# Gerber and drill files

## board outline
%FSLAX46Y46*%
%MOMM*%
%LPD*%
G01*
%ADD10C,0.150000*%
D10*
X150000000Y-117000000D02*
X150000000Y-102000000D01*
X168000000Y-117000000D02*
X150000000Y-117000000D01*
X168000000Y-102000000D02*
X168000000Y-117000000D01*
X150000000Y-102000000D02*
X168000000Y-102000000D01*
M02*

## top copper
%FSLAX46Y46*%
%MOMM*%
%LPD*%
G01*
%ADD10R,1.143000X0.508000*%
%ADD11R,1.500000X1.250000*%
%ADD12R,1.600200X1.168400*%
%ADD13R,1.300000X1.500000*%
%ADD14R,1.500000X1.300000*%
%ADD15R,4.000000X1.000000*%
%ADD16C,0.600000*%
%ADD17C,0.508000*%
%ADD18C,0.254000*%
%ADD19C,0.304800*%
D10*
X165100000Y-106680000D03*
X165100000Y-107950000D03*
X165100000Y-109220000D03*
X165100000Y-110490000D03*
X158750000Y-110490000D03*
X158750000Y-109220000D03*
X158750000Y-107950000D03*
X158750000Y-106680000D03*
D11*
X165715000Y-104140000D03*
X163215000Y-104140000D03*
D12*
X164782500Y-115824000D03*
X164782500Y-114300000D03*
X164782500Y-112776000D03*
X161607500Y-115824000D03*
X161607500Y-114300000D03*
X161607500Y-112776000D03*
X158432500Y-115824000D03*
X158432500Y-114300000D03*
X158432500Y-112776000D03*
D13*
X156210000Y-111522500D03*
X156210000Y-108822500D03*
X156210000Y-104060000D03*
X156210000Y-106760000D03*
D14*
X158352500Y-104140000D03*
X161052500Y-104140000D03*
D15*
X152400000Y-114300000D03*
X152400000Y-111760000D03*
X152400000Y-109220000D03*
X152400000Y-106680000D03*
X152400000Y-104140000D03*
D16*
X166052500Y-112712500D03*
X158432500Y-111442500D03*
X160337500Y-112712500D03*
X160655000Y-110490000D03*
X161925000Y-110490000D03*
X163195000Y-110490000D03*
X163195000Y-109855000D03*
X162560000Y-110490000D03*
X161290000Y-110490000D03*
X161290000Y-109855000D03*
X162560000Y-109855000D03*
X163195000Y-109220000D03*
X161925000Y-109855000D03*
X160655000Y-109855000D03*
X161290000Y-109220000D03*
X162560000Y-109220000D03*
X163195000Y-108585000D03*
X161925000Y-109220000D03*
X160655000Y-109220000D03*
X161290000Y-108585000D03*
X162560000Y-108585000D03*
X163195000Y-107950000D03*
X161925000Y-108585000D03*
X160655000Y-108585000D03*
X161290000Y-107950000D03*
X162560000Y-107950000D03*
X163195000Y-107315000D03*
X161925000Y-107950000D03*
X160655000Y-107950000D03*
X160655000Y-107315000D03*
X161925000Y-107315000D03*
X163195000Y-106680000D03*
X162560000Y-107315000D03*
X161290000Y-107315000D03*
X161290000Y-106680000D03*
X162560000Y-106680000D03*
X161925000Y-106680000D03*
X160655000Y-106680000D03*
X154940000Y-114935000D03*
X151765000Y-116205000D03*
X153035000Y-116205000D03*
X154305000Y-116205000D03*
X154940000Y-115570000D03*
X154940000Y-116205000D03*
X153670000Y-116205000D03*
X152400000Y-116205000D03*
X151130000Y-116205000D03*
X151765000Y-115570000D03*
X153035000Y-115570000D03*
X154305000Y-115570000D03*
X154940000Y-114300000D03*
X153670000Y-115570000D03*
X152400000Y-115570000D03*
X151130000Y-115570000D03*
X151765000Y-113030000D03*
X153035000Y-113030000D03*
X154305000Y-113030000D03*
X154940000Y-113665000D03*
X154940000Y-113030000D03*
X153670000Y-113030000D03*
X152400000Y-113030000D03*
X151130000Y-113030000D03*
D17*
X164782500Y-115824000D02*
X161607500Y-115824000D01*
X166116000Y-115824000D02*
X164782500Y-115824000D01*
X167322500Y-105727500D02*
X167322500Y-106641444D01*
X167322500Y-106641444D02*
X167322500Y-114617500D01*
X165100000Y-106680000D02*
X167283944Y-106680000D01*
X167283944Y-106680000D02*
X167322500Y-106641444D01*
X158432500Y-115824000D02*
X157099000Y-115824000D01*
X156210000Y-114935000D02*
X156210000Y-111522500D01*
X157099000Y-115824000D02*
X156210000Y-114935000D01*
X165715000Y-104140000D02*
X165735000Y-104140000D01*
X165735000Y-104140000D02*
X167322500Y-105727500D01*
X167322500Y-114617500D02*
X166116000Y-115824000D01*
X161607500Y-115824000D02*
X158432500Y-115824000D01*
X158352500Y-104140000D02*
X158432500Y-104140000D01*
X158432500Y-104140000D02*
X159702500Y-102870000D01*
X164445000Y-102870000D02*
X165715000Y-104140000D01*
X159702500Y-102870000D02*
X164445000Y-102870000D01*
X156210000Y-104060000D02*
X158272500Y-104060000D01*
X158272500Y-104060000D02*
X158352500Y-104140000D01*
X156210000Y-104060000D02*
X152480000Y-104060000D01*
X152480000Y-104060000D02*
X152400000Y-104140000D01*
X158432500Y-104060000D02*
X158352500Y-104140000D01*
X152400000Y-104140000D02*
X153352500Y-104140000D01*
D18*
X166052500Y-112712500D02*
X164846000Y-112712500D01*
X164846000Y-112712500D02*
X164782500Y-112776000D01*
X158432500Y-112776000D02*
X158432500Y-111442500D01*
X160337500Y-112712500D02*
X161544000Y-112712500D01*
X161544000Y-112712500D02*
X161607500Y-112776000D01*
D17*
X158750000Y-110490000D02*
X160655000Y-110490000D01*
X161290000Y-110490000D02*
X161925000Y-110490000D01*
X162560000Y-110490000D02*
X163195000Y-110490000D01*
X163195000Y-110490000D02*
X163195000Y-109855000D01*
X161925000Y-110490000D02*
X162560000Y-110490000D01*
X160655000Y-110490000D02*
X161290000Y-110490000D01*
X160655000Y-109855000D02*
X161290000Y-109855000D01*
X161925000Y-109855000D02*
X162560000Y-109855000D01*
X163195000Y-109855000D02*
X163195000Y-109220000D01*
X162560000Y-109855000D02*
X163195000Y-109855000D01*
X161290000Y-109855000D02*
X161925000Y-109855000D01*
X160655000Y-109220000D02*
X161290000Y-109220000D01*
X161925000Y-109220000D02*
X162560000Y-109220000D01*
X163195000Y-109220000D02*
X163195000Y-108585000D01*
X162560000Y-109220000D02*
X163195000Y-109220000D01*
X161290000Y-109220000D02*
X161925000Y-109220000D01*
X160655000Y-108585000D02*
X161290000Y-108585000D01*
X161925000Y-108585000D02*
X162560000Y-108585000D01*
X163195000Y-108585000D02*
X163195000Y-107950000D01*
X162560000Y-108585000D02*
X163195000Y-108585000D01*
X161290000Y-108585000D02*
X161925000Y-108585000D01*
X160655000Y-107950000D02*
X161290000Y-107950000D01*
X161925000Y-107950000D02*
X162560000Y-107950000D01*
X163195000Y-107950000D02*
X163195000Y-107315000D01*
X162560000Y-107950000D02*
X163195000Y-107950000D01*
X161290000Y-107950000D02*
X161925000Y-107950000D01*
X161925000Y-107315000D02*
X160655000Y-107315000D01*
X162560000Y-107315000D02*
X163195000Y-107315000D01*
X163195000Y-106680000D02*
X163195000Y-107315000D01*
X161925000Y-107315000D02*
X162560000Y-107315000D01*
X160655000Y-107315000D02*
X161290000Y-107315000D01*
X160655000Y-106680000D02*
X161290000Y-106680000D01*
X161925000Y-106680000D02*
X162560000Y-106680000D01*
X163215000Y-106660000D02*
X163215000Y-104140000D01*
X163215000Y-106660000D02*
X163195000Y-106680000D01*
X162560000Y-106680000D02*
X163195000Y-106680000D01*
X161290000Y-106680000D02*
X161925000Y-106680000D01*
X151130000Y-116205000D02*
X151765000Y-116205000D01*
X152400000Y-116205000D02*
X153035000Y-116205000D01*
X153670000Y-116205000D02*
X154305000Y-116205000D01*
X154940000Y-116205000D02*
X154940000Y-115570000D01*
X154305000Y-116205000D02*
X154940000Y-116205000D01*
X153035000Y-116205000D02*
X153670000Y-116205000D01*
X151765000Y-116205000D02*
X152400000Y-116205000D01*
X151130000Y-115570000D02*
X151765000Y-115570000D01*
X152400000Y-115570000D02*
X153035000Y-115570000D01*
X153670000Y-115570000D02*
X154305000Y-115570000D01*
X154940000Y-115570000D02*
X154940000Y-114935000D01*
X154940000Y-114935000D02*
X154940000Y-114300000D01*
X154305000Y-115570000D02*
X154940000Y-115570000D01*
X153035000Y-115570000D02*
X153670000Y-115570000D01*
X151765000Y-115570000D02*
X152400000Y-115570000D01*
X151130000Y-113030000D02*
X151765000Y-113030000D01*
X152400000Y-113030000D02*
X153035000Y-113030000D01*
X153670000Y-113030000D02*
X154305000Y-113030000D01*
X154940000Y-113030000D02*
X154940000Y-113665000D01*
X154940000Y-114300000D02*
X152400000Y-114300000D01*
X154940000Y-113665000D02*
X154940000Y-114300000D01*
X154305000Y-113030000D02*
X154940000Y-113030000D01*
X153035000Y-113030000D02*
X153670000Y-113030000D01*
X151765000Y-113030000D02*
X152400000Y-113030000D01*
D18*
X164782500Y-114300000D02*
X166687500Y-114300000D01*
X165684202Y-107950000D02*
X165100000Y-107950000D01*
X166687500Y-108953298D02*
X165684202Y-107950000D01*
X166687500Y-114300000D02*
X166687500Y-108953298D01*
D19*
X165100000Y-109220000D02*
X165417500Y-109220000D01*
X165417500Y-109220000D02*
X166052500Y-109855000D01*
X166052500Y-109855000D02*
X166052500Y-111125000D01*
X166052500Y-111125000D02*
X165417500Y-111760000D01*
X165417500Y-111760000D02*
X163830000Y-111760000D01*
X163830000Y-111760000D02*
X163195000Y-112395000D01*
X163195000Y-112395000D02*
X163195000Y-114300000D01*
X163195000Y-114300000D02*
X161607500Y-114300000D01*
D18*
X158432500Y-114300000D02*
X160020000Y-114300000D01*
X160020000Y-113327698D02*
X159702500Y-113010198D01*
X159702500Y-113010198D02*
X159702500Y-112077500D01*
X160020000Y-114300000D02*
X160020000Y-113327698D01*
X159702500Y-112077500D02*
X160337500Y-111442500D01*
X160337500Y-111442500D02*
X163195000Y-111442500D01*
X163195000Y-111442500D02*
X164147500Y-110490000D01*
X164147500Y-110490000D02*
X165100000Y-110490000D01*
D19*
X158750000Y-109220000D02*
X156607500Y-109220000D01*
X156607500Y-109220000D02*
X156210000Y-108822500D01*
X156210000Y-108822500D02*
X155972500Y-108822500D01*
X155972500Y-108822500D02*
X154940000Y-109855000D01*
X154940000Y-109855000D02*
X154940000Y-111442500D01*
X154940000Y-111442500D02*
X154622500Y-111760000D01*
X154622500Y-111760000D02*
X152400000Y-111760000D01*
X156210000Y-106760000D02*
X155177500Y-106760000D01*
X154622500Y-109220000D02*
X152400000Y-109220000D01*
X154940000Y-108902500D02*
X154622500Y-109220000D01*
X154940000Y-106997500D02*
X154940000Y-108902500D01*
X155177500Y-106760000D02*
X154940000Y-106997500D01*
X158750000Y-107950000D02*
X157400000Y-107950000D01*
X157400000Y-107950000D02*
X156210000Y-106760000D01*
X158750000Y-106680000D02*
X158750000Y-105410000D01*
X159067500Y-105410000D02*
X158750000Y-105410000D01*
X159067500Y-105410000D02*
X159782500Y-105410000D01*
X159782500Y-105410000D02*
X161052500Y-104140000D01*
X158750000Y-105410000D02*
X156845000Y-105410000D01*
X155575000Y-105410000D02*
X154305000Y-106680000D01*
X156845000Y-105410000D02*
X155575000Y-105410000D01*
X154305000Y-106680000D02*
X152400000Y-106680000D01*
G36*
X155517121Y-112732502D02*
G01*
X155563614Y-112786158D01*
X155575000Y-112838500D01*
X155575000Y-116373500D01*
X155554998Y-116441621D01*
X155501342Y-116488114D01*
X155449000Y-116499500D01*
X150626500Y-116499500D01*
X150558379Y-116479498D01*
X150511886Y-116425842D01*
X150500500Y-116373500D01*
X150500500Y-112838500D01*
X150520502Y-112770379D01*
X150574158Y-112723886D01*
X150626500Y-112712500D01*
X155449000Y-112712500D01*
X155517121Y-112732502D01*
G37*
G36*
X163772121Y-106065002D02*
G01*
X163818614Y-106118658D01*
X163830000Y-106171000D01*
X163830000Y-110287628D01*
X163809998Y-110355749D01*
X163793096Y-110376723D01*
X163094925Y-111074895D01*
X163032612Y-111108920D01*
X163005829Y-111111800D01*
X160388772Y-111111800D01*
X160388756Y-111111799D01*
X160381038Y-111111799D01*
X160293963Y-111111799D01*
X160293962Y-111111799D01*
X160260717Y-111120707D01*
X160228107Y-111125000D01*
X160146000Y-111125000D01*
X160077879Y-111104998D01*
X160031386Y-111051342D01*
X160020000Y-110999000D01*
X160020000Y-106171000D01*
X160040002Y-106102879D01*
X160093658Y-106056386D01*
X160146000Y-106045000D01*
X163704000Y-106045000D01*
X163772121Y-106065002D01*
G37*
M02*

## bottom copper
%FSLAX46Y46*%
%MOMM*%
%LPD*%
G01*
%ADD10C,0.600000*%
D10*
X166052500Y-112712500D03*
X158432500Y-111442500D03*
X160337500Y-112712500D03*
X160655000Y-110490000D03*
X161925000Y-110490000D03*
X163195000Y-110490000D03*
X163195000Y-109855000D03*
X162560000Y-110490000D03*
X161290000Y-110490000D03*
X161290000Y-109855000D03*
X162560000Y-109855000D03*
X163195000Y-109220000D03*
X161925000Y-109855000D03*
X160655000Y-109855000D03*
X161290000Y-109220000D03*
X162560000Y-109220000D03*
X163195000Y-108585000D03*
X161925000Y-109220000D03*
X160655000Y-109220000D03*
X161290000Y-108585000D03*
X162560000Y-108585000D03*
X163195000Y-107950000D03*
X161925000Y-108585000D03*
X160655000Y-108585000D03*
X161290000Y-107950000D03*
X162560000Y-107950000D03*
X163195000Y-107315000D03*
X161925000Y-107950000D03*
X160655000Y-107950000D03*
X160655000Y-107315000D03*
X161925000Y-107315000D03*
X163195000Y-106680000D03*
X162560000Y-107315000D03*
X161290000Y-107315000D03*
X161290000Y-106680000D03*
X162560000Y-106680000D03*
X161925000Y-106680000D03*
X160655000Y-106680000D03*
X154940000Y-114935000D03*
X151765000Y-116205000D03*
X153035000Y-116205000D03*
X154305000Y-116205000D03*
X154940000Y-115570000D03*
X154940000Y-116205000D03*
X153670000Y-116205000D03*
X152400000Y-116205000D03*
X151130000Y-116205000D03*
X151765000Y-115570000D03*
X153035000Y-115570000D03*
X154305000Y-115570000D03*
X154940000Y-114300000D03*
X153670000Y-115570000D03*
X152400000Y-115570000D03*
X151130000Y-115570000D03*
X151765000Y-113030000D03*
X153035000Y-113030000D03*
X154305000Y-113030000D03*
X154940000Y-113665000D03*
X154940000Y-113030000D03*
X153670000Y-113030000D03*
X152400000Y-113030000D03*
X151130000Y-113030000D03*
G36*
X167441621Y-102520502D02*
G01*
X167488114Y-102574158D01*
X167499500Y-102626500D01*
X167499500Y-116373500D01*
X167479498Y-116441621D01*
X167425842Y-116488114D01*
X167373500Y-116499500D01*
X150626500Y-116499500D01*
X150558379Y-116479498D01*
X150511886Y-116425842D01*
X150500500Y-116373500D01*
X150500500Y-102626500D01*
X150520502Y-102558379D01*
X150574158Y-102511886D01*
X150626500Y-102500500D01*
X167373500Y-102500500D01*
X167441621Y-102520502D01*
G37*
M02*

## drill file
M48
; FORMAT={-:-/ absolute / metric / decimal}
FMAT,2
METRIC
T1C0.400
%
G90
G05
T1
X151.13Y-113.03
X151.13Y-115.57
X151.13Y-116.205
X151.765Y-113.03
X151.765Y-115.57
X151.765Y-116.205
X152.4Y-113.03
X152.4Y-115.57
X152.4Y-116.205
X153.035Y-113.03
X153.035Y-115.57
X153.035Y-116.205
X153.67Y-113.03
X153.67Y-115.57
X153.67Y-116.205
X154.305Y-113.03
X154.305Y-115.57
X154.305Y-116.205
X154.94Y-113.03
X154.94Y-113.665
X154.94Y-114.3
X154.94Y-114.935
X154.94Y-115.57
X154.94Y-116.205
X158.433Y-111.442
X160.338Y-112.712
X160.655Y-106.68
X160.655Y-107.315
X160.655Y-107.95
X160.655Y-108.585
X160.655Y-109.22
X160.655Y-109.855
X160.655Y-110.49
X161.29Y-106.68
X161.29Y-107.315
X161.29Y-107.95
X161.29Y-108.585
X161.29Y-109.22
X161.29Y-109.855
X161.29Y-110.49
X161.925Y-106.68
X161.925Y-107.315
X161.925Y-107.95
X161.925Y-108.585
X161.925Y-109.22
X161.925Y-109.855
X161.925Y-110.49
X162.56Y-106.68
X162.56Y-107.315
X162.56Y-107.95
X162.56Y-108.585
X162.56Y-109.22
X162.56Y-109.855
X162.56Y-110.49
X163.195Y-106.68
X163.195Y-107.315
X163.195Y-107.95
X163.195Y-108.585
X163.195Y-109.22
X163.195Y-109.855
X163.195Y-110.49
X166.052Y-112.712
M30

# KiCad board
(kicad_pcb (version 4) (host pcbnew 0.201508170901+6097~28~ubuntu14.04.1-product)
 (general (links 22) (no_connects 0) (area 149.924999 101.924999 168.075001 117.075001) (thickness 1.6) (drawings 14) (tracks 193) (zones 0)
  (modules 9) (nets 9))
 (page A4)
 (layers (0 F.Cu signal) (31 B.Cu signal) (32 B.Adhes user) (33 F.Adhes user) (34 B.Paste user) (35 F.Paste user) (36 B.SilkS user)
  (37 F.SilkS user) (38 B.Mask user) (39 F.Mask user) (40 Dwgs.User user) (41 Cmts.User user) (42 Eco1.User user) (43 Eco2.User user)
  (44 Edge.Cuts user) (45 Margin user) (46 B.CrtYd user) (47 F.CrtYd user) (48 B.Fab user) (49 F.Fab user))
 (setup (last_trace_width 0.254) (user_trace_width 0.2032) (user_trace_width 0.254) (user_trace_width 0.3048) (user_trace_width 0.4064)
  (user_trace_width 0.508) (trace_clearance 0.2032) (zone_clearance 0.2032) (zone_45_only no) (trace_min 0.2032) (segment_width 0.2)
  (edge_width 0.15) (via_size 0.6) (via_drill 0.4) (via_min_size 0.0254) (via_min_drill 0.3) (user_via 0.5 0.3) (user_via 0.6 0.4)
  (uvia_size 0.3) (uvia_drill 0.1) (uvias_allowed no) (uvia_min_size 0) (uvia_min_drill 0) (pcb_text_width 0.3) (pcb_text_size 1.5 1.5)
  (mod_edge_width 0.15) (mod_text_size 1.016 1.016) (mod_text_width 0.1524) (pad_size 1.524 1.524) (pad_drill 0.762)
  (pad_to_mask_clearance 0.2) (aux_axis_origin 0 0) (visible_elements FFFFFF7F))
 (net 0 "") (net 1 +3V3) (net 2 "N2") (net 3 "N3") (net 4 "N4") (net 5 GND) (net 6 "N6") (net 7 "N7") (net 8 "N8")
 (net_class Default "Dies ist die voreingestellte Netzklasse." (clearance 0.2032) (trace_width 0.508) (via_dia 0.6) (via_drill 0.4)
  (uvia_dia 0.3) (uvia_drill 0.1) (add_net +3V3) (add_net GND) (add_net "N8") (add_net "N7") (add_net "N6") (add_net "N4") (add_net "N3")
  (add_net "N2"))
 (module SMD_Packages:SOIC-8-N (layer F.Cu) (at 161.925 108.585 270)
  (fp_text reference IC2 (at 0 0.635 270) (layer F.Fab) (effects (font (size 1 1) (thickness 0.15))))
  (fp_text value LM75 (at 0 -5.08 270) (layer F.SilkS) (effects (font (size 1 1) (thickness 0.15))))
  (pad 8 smd rect (at -1.905 -3.175 270) (size 0.508 1.143) (layers F.Cu F.Paste F.Mask) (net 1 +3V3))
  (pad 7 smd rect (at -0.635 -3.175 270) (size 0.508 1.143) (layers F.Cu F.Paste F.Mask) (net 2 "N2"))
  (pad 6 smd rect (at 0.635 -3.175 270) (size 0.508 1.143) (layers F.Cu F.Paste F.Mask) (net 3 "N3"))
  (pad 5 smd rect (at 1.905 -3.175 270) (size 0.508 1.143) (layers F.Cu F.Paste F.Mask) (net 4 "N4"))
  (pad 4 smd rect (at 1.905 3.175 270) (size 0.508 1.143) (layers F.Cu F.Paste F.Mask) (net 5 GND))
  (pad 3 smd rect (at 0.635 3.175 270) (size 0.508 1.143) (layers F.Cu F.Paste F.Mask) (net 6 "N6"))
  (pad 2 smd rect (at -0.635 3.175 270) (size 0.508 1.143) (layers F.Cu F.Paste F.Mask) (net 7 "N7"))
  (pad 1 smd rect (at -1.905 3.175 270) (size 0.508 1.143) (layers F.Cu F.Paste F.Mask) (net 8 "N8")))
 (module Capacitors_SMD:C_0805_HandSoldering (layer F.Cu) (at 164.465 104.14 180)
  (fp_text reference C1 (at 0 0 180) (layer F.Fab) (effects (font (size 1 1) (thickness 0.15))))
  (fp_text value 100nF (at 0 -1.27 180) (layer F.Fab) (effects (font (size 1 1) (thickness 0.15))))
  (pad 1 smd rect (at -1.25 0 180) (size 1.5 1.25) (layers F.Cu F.Paste F.Mask) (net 1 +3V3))
  (pad 2 smd rect (at 1.25 0 180) (size 1.5 1.25) (layers F.Cu F.Paste F.Mask) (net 5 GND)))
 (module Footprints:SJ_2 (layer F.Cu) (at 164.7825 114.3 90)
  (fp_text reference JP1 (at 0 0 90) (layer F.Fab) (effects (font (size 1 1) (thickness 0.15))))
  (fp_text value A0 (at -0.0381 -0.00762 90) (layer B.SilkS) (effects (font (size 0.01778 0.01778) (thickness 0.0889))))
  (pad 1 smd rect (at -1.524 0 90) (size 1.1684 1.6002) (layers F.Cu F.Paste F.Mask) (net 1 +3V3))
  (pad 2 smd rect (at 0 0 90) (size 1.1684 1.6002) (layers F.Cu F.Paste F.Mask) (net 2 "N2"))
  (pad 3 smd rect (at 1.524 0 90) (size 1.1684 1.6002) (layers F.Cu F.Paste F.Mask) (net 5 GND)))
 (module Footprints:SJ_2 (layer F.Cu) (at 161.6075 114.3 90)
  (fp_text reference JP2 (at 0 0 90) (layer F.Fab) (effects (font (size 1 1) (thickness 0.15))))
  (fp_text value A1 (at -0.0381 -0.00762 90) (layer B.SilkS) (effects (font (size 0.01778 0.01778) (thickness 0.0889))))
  (pad 1 smd rect (at -1.524 0 90) (size 1.1684 1.6002) (layers F.Cu F.Paste F.Mask) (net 1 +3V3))
  (pad 2 smd rect (at 0 0 90) (size 1.1684 1.6002) (layers F.Cu F.Paste F.Mask) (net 3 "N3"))
  (pad 3 smd rect (at 1.524 0 90) (size 1.1684 1.6002) (layers F.Cu F.Paste F.Mask) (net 5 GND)))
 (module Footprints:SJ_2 (layer F.Cu) (at 158.4325 114.3 90)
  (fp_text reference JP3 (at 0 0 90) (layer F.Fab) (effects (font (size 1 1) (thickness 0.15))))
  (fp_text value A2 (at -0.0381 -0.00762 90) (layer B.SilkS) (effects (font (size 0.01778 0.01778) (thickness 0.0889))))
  (pad 1 smd rect (at -1.524 0 90) (size 1.1684 1.6002) (layers F.Cu F.Paste F.Mask) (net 1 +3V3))
  (pad 2 smd rect (at 0 0 90) (size 1.1684 1.6002) (layers F.Cu F.Paste F.Mask) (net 4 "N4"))
  (pad 3 smd rect (at 1.524 0 90) (size 1.1684 1.6002) (layers F.Cu F.Paste F.Mask) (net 5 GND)))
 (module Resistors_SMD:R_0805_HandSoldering (layer F.Cu) (at 156.21 110.1725 90)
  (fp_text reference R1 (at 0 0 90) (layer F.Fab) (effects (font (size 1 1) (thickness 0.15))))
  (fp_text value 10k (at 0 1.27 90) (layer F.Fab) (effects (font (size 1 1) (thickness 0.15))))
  (pad 1 smd rect (at -1.35 0 90) (size 1.5 1.3) (layers F.Cu F.Paste F.Mask) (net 1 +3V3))
  (pad 2 smd rect (at 1.35 0 90) (size 1.5 1.3) (layers F.Cu F.Paste F.Mask) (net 6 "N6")))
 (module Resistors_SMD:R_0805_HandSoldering (layer F.Cu) (at 156.21 105.41 270)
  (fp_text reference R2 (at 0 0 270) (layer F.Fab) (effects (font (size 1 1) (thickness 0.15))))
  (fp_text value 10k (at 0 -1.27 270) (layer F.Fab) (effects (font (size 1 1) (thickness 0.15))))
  (pad 1 smd rect (at -1.35 0 270) (size 1.5 1.3) (layers F.Cu F.Paste F.Mask) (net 1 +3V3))
  (pad 2 smd rect (at 1.35 0 270) (size 1.5 1.3) (layers F.Cu F.Paste F.Mask) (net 7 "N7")))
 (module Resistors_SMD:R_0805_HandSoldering (layer F.Cu) (at 159.7025 104.14)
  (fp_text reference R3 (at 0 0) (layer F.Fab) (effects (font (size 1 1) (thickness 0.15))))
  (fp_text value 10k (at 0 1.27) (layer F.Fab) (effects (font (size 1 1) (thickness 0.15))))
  (pad 1 smd rect (at -1.35 0) (size 1.5 1.3) (layers F.Cu F.Paste F.Mask) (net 1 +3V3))
  (pad 2 smd rect (at 1.35 0) (size 1.5 1.3) (layers F.Cu F.Paste F.Mask) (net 8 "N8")))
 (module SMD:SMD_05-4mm (layer F.Cu) (at 152.4 104.14)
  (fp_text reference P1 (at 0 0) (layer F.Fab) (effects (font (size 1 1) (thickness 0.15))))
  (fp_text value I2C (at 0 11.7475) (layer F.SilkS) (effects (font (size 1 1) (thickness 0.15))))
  (pad 5 connect rect (at 0 10.16) (size 4 1) (layers F.Cu F.Mask) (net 5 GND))
  (pad 4 connect rect (at 0 7.62) (size 4 1) (layers F.Cu F.Mask) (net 6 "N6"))
  (pad 3 connect rect (at 0 5.08) (size 4 1) (layers F.Cu F.Mask) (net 7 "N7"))
  (pad 2 connect rect (at 0 2.54) (size 4 1) (layers F.Cu F.Mask) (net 8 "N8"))
  (pad 1 connect rect (at 0 0) (size 4 1) (layers F.Cu F.Mask) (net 1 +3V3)))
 (gr_line (start 150 117) (end 150 102) (angle 90) (layer Edge.Cuts) (width 0.15))
 (gr_line (start 168 117) (end 150 117) (angle 90) (layer Edge.Cuts) (width 0.15))
 (gr_line (start 168 102) (end 168 117) (angle 90) (layer Edge.Cuts) (width 0.15))
 (gr_line (start 150 102) (end 168 102) (angle 90) (layer Edge.Cuts) (width 0.15))
 (segment (start 164.7825 115.824) (end 161.6075 115.824) (width 0.508) (layer F.Cu) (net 1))
 (segment (start 166.116 115.824) (end 164.7825 115.824) (width 0.508) (layer F.Cu) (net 1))
 (segment (start 167.3225 105.7275) (end 167.3225 106.641444) (width 0.508) (layer F.Cu) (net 1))
 (segment (start 167.3225 106.641444) (end 167.3225 114.6175) (width 0.508) (layer F.Cu) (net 1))
 (segment (start 165.1 106.68) (end 167.283944 106.68) (width 0.508) (layer F.Cu) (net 1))
 (segment (start 167.283944 106.68) (end 167.3225 106.641444) (width 0.508) (layer F.Cu) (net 1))
 (segment (start 158.4325 115.824) (end 157.099 115.824) (width 0.508) (layer F.Cu) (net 1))
 (segment (start 156.21 114.935) (end 156.21 111.5225) (width 0.508) (layer F.Cu) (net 1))
 (segment (start 157.099 115.824) (end 156.21 114.935) (width 0.508) (layer F.Cu) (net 1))
 (segment (start 165.715 104.14) (end 165.735 104.14) (width 0.508) (layer F.Cu) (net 1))
 (segment (start 165.735 104.14) (end 167.3225 105.7275) (width 0.508) (layer F.Cu) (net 1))
 (segment (start 167.3225 114.6175) (end 166.116 115.824) (width 0.508) (layer F.Cu) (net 1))
 (segment (start 161.6075 115.824) (end 158.4325 115.824) (width 0.508) (layer F.Cu) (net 1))
 (segment (start 158.3525 104.14) (end 158.4325 104.14) (width 0.508) (layer F.Cu) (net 1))
 (segment (start 158.4325 104.14) (end 159.7025 102.87) (width 0.508) (layer F.Cu) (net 1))
 (segment (start 164.445 102.87) (end 165.715 104.14) (width 0.508) (layer F.Cu) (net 1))
 (segment (start 159.7025 102.87) (end 164.445 102.87) (width 0.508) (layer F.Cu) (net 1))
 (segment (start 156.21 104.06) (end 158.2725 104.06) (width 0.508) (layer F.Cu) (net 1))
 (segment (start 158.2725 104.06) (end 158.3525 104.14) (width 0.508) (layer F.Cu) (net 1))
 (segment (start 156.21 104.06) (end 152.48 104.06) (width 0.508) (layer F.Cu) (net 1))
 (segment (start 152.48 104.06) (end 152.4 104.14) (width 0.508) (layer F.Cu) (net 1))
 (segment (start 158.4325 104.06) (end 158.3525 104.14) (width 0.508) (layer F.Cu) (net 1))
 (segment (start 152.4 104.14) (end 153.3525 104.14) (width 0.508) (layer F.Cu) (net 1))
 (via (at 166.0525 112.7125) (size 0.6) (drill 0.4) (layers F.Cu B.Cu) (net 5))
 (segment (start 166.0525 112.7125) (end 164.846 112.7125) (width 0.254) (layer F.Cu) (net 5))
 (segment (start 164.846 112.7125) (end 164.7825 112.776) (width 0.254) (layer F.Cu) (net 5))
 (segment (start 158.4325 112.776) (end 158.4325 111.4425) (width 0.254) (layer F.Cu) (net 5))
 (via (at 158.4325 111.4425) (size 0.6) (drill 0.4) (layers F.Cu B.Cu) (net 5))
 (via (at 160.3375 112.7125) (size 0.6) (drill 0.4) (layers F.Cu B.Cu) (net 5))
 (segment (start 160.3375 112.7125) (end 161.544 112.7125) (width 0.254) (layer F.Cu) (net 5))
 (segment (start 161.544 112.7125) (end 161.6075 112.776) (width 0.254) (layer F.Cu) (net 5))
 (segment (start 158.75 110.49) (end 160.655 110.49) (width 0.508) (layer F.Cu) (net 5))
 (via (at 160.655 110.49) (size 0.6) (drill 0.4) (layers F.Cu B.Cu) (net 5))
 (segment (start 161.29 110.49) (end 161.925 110.49) (width 0.508) (layer F.Cu) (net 5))
 (via (at 161.925 110.49) (size 0.6) (drill 0.4) (layers F.Cu B.Cu) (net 5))
 (segment (start 162.56 110.49) (end 163.195 110.49) (width 0.508) (layer F.Cu) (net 5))
 (via (at 163.195 110.49) (size 0.6) (drill 0.4) (layers F.Cu B.Cu) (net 5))
 (via (at 163.195 109.855) (size 0.6) (drill 0.4) (layers F.Cu B.Cu) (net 5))
 (segment (start 163.195 110.49) (end 163.195 109.855) (width 0.508) (layer F.Cu) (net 5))
 (via (at 162.56 110.49) (size 0.6) (drill 0.4) (layers F.Cu B.Cu) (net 5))
 (segment (start 161.925 110.49) (end 162.56 110.49) (width 0.508) (layer F.Cu) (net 5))
 (via (at 161.29 110.49) (size 0.6) (drill 0.4) (layers F.Cu B.Cu) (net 5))
 (segment (start 160.655 110.49) (end 161.29 110.49) (width 0.508) (layer F.Cu) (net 5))
 (segment (start 160.655 109.855) (end 161.29 109.855) (width 0.508) (layer F.Cu) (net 5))
 (via (at 161.29 109.855) (size 0.6) (drill 0.4) (layers F.Cu B.Cu) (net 5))
 (segment (start 161.925 109.855) (end 162.56 109.855) (width 0.508) (layer F.Cu) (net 5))
 (via (at 162.56 109.855) (size 0.6) (drill 0.4) (layers F.Cu B.Cu) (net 5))
 (segment (start 163.195 109.855) (end 163.195 109.22) (width 0.508) (layer F.Cu) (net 5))
 (via (at 163.195 109.22) (size 0.6) (drill 0.4) (layers F.Cu B.Cu) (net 5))
 (segment (start 162.56 109.855) (end 163.195 109.855) (width 0.508) (layer F.Cu) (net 5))
 (via (at 161.925 109.855) (size 0.6) (drill 0.4) (layers F.Cu B.Cu) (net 5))
 (segment (start 161.29 109.855) (end 161.925 109.855) (width 0.508) (layer F.Cu) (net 5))
 (via (at 160.655 109.855) (size 0.6) (drill 0.4) (layers F.Cu B.Cu) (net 5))
 (segment (start 160.655 109.22) (end 161.29 109.22) (width 0.508) (layer F.Cu) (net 5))
 (via (at 161.29 109.22) (size 0.6) (drill 0.4) (layers F.Cu B.Cu) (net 5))
 (segment (start 161.925 109.22) (end 162.56 109.22) (width 0.508) (layer F.Cu) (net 5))
 (via (at 162.56 109.22) (size 0.6) (drill 0.4) (layers F.Cu B.Cu) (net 5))
 (segment (start 163.195 109.22) (end 163.195 108.585) (width 0.508) (layer F.Cu) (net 5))
 (via (at 163.195 108.585) (size 0.6) (drill 0.4) (layers F.Cu B.Cu) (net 5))
 (segment (start 162.56 109.22) (end 163.195 109.22) (width 0.508) (layer F.Cu) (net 5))
 (via (at 161.925 109.22) (size 0.6) (drill 0.4) (layers F.Cu B.Cu) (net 5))
 (segment (start 161.29 109.22) (end 161.925 109.22) (width 0.508) (layer F.Cu) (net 5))
 (via (at 160.655 109.22) (size 0.6) (drill 0.4) (layers F.Cu B.Cu) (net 5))
 (segment (start 160.655 108.585) (end 161.29 108.585) (width 0.508) (layer F.Cu) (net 5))
 (via (at 161.29 108.585) (size 0.6) (drill 0.4) (layers F.Cu B.Cu) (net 5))
 (segment (start 161.925 108.585) (end 162.56 108.585) (width 0.508) (layer F.Cu) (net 5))
 (via (at 162.56 108.585) (size 0.6) (drill 0.4) (layers F.Cu B.Cu) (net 5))
 (segment (start 163.195 108.585) (end 163.195 107.95) (width 0.508) (layer F.Cu) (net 5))
 (via (at 163.195 107.95) (size 0.6) (drill 0.4) (layers F.Cu B.Cu) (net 5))
 (segment (start 162.56 108.585) (end 163.195 108.585) (width 0.508) (layer F.Cu) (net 5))
 (via (at 161.925 108.585) (size 0.6) (drill 0.4) (layers F.Cu B.Cu) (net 5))
 (segment (start 161.29 108.585) (end 161.925 108.585) (width 0.508) (layer F.Cu) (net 5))
 (via (at 160.655 108.585) (size 0.6) (drill 0.4) (layers F.Cu B.Cu) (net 5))
 (segment (start 160.655 107.95) (end 161.29 107.95) (width 0.508) (layer F.Cu) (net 5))
 (via (at 161.29 107.95) (size 0.6) (drill 0.4) (layers F.Cu B.Cu) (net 5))
 (segment (start 161.925 107.95) (end 162.56 107.95) (width 0.508) (layer F.Cu) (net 5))
 (via (at 162.56 107.95) (size 0.6) (drill 0.4) (layers F.Cu B.Cu) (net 5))
 (segment (start 163.195 107.95) (end 163.195 107.315) (width 0.508) (layer F.Cu) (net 5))
 (via (at 163.195 107.315) (size 0.6) (drill 0.4) (layers F.Cu B.Cu) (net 5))
 (segment (start 162.56 107.95) (end 163.195 107.95) (width 0.508) (layer F.Cu) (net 5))
 (via (at 161.925 107.95) (size 0.6) (drill 0.4) (layers F.Cu B.Cu) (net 5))
 (segment (start 161.29 107.95) (end 161.925 107.95) (width 0.508) (layer F.Cu) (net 5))
 (via (at 160.655 107.95) (size 0.6) (drill 0.4) (layers F.Cu B.Cu) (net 5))
 (via (at 160.655 107.315) (size 0.6) (drill 0.4) (layers F.Cu B.Cu) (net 5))
 (segment (start 161.925 107.315) (end 160.655 107.315) (width 0.508) (layer F.Cu) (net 5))
 (via (at 161.925 107.315) (size 0.6) (drill 0.4) (layers F.Cu B.Cu) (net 5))
 (segment (start 162.56 107.315) (end 163.195 107.315) (width 0.508) (layer F.Cu) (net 5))
 (via (at 163.195 106.68) (size 0.6) (drill 0.4) (layers F.Cu B.Cu) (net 5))
 (segment (start 163.195 106.68) (end 163.195 107.315) (width 0.508) (layer F.Cu) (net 5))
 (via (at 162.56 107.315) (size 0.6) (drill 0.4) (layers F.Cu B.Cu) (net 5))
 (segment (start 161.925 107.315) (end 162.56 107.315) (width 0.508) (layer F.Cu) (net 5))
 (via (at 161.29 107.315) (size 0.6) (drill 0.4) (layers F.Cu B.Cu) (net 5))
 (segment (start 160.655 107.315) (end 161.29 107.315) (width 0.508) (layer F.Cu) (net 5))
 (segment (start 160.655 106.68) (end 161.29 106.68) (width 0.508) (layer F.Cu) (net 5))
 (via (at 161.29 106.68) (size 0.6) (drill 0.4) (layers F.Cu B.Cu) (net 5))
 (segment (start 161.925 106.68) (end 162.56 106.68) (width 0.508) (layer F.Cu) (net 5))
 (via (at 162.56 106.68) (size 0.6) (drill 0.4) (layers F.Cu B.Cu) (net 5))
 (segment (start 163.215 106.66) (end 163.215 104.14) (width 0.508) (layer F.Cu) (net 5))
 (segment (start 163.215 106.66) (end 163.195 106.68) (width 0.508) (layer F.Cu) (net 5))
 (segment (start 162.56 106.68) (end 163.195 106.68) (width 0.508) (layer F.Cu) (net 5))
 (via (at 161.925 106.68) (size 0.6) (drill 0.4) (layers F.Cu B.Cu) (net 5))
 (segment (start 161.29 106.68) (end 161.925 106.68) (width 0.508) (layer F.Cu) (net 5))
 (via (at 160.655 106.68) (size 0.6) (drill 0.4) (layers F.Cu B.Cu) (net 5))
 (via (at 154.94 114.935) (size 0.6) (drill 0.4) (layers F.Cu B.Cu) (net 5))
 (segment (start 151.13 116.205) (end 151.765 116.205) (width 0.508) (layer F.Cu) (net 5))
 (via (at 151.765 116.205) (size 0.6) (drill 0.4) (layers F.Cu B.Cu) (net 5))
 (segment (start 152.4 116.205) (end 153.035 116.205) (width 0.508) (layer F.Cu) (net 5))
 (via (at 153.035 116.205) (size 0.6) (drill 0.4) (layers F.Cu B.Cu) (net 5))
 (segment (start 153.67 116.205) (end 154.305 116.205) (width 0.508) (layer F.Cu) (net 5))
 (via (at 154.305 116.205) (size 0.6) (drill 0.4) (layers F.Cu B.Cu) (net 5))
 (segment (start 154.94 116.205) (end 154.94 115.57) (width 0.508) (layer F.Cu) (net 5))
 (via (at 154.94 115.57) (size 0.6) (drill 0.4) (layers F.Cu B.Cu) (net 5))
 (via (at 154.94 116.205) (size 0.6) (drill 0.4) (layers F.Cu B.Cu) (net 5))
 (segment (start 154.305 116.205) (end 154.94 116.205) (width 0.508) (layer F.Cu) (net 5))
 (via (at 153.67 116.205) (size 0.6) (drill 0.4) (layers F.Cu B.Cu) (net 5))
 (segment (start 153.035 116.205) (end 153.67 116.205) (width 0.508) (layer F.Cu) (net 5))
 (via (at 152.4 116.205) (size 0.6) (drill 0.4) (layers F.Cu B.Cu) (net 5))
 (segment (start 151.765 116.205) (end 152.4 116.205) (width 0.508) (layer F.Cu) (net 5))
 (via (at 151.13 116.205) (size 0.6) (drill 0.4) (layers F.Cu B.Cu) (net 5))
 (segment (start 151.13 115.57) (end 151.765 115.57) (width 0.508) (layer F.Cu) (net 5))
 (via (at 151.765 115.57) (size 0.6) (drill 0.4) (layers F.Cu B.Cu) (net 5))
 (segment (start 152.4 115.57) (end 153.035 115.57) (width 0.508) (layer F.Cu) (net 5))
 (via (at 153.035 115.57) (size 0.6) (drill 0.4) (layers F.Cu B.Cu) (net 5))
 (segment (start 153.67 115.57) (end 154.305 115.57) (width 0.508) (layer F.Cu) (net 5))
 (via (at 154.305 115.57) (size 0.6) (drill 0.4) (layers F.Cu B.Cu) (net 5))
 (segment (start 154.94 115.57) (end 154.94 114.935) (width 0.508) (layer F.Cu) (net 5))
 (via (at 154.94 114.3) (size 0.6) (drill 0.4) (layers F.Cu B.Cu) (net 5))
 (segment (start 154.94 114.935) (end 154.94 114.3) (width 0.508) (layer F.Cu) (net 5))
 (segment (start 154.305 115.57) (end 154.94 115.57) (width 0.508) (layer F.Cu) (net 5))
 (via (at 153.67 115.57) (size 0.6) (drill 0.4) (layers F.Cu B.Cu) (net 5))
 (segment (start 153.035 115.57) (end 153.67 115.57) (width 0.508) (layer F.Cu) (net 5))
 (via (at 152.4 115.57) (size 0.6) (drill 0.4) (layers F.Cu B.Cu) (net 5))
 (segment (start 151.765 115.57) (end 152.4 115.57) (width 0.508) (layer F.Cu) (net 5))
 (via (at 151.13 115.57) (size 0.6) (drill 0.4) (layers F.Cu B.Cu) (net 5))
 (segment (start 151.13 113.03) (end 151.765 113.03) (width 0.508) (layer F.Cu) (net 5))
 (via (at 151.765 113.03) (size 0.6) (drill 0.4) (layers F.Cu B.Cu) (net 5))
 (segment (start 152.4 113.03) (end 153.035 113.03) (width 0.508) (layer F.Cu) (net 5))
 (via (at 153.035 113.03) (size 0.6) (drill 0.4) (layers F.Cu B.Cu) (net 5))
 (segment (start 153.67 113.03) (end 154.305 113.03) (width 0.508) (layer F.Cu) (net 5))
 (via (at 154.305 113.03) (size 0.6) (drill 0.4) (layers F.Cu B.Cu) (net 5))
 (segment (start 154.94 113.03) (end 154.94 113.665) (width 0.508) (layer F.Cu) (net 5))
 (via (at 154.94 113.665) (size 0.6) (drill 0.4) (layers F.Cu B.Cu) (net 5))
 (segment (start 154.94 114.3) (end 152.4 114.3) (width 0.508) (layer F.Cu) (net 5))
 (segment (start 154.94 113.665) (end 154.94 114.3) (width 0.508) (layer F.Cu) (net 5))
 (via (at 154.94 113.03) (size 0.6) (drill 0.4) (layers F.Cu B.Cu) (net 5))
 (segment (start 154.305 113.03) (end 154.94 113.03) (width 0.508) (layer F.Cu) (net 5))
 (via (at 153.67 113.03) (size 0.6) (drill 0.4) (layers F.Cu B.Cu) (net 5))
 (segment (start 153.035 113.03) (end 153.67 113.03) (width 0.508) (layer F.Cu) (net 5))
 (via (at 152.4 113.03) (size 0.6) (drill 0.4) (layers F.Cu B.Cu) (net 5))
 (segment (start 151.765 113.03) (end 152.4 113.03) (width 0.508) (layer F.Cu) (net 5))
 (via (at 151.13 113.03) (size 0.6) (drill 0.4) (layers F.Cu B.Cu) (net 5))
 (segment (start 164.7825 114.3) (end 166.6875 114.3) (width 0.254) (layer F.Cu) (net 2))
 (segment (start 165.684202 107.95) (end 165.1 107.95) (width 0.254) (layer F.Cu) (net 2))
 (segment (start 166.6875 108.953298) (end 165.684202 107.95) (width 0.254) (layer F.Cu) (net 2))
 (segment (start 166.6875 114.3) (end 166.6875 108.953298) (width 0.254) (layer F.Cu) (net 2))
 (segment (start 165.1 109.22) (end 165.4175 109.22) (width 0.3048) (layer F.Cu) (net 3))
 (segment (start 165.4175 109.22) (end 166.0525 109.855) (width 0.3048) (layer F.Cu) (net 3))
 (segment (start 166.0525 109.855) (end 166.0525 111.125) (width 0.3048) (layer F.Cu) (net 3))
 (segment (start 166.0525 111.125) (end 165.4175 111.76) (width 0.3048) (layer F.Cu) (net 3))
 (segment (start 165.4175 111.76) (end 163.83 111.76) (width 0.3048) (layer F.Cu) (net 3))
 (segment (start 163.83 111.76) (end 163.195 112.395) (width 0.3048) (layer F.Cu) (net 3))
 (segment (start 163.195 112.395) (end 163.195 114.3) (width 0.3048) (layer F.Cu) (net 3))
 (segment (start 163.195 114.3) (end 161.6075 114.3) (width 0.3048) (layer F.Cu) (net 3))
 (segment (start 158.4325 114.3) (end 160.02 114.3) (width 0.254) (layer F.Cu) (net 4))
 (segment (start 160.02 113.327698) (end 159.7025 113.010198) (width 0.254) (layer F.Cu) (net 4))
 (segment (start 159.7025 113.010198) (end 159.7025 112.0775) (width 0.254) (layer F.Cu) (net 4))
 (segment (start 160.02 114.3) (end 160.02 113.327698) (width 0.254) (layer F.Cu) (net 4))
 (segment (start 159.7025 112.0775) (end 160.3375 111.4425) (width 0.254) (layer F.Cu) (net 4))
 (segment (start 160.3375 111.4425) (end 163.195 111.4425) (width 0.254) (layer F.Cu) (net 4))
 (segment (start 163.195 111.4425) (end 164.1475 110.49) (width 0.254) (layer F.Cu) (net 4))
 (segment (start 164.1475 110.49) (end 165.1 110.49) (width 0.254) (layer F.Cu) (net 4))
 (segment (start 158.75 109.22) (end 156.6075 109.22) (width 0.3048) (layer F.Cu) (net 6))
 (segment (start 156.6075 109.22) (end 156.21 108.8225) (width 0.3048) (layer F.Cu) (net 6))
 (segment (start 156.21 108.8225) (end 155.9725 108.8225) (width 0.3048) (layer F.Cu) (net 6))
 (segment (start 155.9725 108.8225) (end 154.94 109.855) (width 0.3048) (layer F.Cu) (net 6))
 (segment (start 154.94 109.855) (end 154.94 111.4425) (width 0.3048) (layer F.Cu) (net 6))
 (segment (start 154.94 111.4425) (end 154.6225 111.76) (width 0.3048) (layer F.Cu) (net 6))
 (segment (start 154.6225 111.76) (end 152.4 111.76) (width 0.3048) (layer F.Cu) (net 6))
 (segment (start 156.21 106.76) (end 155.1775 106.76) (width 0.3048) (layer F.Cu) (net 7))
 (segment (start 154.6225 109.22) (end 152.4 109.22) (width 0.3048) (layer F.Cu) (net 7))
 (segment (start 154.94 108.9025) (end 154.6225 109.22) (width 0.3048) (layer F.Cu) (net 7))
 (segment (start 154.94 106.9975) (end 154.94 108.9025) (width 0.3048) (layer F.Cu) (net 7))
 (segment (start 155.1775 106.76) (end 154.94 106.9975) (width 0.3048) (layer F.Cu) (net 7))
 (segment (start 158.75 107.95) (end 157.4 107.95) (width 0.3048) (layer F.Cu) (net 7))
 (segment (start 157.4 107.95) (end 156.21 106.76) (width 0.3048) (layer F.Cu) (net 7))
 (segment (start 158.75 106.68) (end 158.75 105.41) (width 0.3048) (layer F.Cu) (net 8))
 (segment (start 159.0675 105.41) (end 158.75 105.41) (width 0.3048) (layer F.Cu) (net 8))
 (segment (start 159.0675 105.41) (end 159.7825 105.41) (width 0.3048) (layer F.Cu) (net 8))
 (segment (start 159.7825 105.41) (end 161.0525 104.14) (width 0.3048) (layer F.Cu) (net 8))
 (segment (start 158.75 105.41) (end 156.845 105.41) (width 0.3048) (layer F.Cu) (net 8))
 (segment (start 155.575 105.41) (end 154.305 106.68) (width 0.3048) (layer F.Cu) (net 8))
 (segment (start 156.845 105.41) (end 155.575 105.41) (width 0.3048) (layer F.Cu) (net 8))
 (segment (start 154.305 106.68) (end 152.4 106.68) (width 0.3048) (layer F.Cu) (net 8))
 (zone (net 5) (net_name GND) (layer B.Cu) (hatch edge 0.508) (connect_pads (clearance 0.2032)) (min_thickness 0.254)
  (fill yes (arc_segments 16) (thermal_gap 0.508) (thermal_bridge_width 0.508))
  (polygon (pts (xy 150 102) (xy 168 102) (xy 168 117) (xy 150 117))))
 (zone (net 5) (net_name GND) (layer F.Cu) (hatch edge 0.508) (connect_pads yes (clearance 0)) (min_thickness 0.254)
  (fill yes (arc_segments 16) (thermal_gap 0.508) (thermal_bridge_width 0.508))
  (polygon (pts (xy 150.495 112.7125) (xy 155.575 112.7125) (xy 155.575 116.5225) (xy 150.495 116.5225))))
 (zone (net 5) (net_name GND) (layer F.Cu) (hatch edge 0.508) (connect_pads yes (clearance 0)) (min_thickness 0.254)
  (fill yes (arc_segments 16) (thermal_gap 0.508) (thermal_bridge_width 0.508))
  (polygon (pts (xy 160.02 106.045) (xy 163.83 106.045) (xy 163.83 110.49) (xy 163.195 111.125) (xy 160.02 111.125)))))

